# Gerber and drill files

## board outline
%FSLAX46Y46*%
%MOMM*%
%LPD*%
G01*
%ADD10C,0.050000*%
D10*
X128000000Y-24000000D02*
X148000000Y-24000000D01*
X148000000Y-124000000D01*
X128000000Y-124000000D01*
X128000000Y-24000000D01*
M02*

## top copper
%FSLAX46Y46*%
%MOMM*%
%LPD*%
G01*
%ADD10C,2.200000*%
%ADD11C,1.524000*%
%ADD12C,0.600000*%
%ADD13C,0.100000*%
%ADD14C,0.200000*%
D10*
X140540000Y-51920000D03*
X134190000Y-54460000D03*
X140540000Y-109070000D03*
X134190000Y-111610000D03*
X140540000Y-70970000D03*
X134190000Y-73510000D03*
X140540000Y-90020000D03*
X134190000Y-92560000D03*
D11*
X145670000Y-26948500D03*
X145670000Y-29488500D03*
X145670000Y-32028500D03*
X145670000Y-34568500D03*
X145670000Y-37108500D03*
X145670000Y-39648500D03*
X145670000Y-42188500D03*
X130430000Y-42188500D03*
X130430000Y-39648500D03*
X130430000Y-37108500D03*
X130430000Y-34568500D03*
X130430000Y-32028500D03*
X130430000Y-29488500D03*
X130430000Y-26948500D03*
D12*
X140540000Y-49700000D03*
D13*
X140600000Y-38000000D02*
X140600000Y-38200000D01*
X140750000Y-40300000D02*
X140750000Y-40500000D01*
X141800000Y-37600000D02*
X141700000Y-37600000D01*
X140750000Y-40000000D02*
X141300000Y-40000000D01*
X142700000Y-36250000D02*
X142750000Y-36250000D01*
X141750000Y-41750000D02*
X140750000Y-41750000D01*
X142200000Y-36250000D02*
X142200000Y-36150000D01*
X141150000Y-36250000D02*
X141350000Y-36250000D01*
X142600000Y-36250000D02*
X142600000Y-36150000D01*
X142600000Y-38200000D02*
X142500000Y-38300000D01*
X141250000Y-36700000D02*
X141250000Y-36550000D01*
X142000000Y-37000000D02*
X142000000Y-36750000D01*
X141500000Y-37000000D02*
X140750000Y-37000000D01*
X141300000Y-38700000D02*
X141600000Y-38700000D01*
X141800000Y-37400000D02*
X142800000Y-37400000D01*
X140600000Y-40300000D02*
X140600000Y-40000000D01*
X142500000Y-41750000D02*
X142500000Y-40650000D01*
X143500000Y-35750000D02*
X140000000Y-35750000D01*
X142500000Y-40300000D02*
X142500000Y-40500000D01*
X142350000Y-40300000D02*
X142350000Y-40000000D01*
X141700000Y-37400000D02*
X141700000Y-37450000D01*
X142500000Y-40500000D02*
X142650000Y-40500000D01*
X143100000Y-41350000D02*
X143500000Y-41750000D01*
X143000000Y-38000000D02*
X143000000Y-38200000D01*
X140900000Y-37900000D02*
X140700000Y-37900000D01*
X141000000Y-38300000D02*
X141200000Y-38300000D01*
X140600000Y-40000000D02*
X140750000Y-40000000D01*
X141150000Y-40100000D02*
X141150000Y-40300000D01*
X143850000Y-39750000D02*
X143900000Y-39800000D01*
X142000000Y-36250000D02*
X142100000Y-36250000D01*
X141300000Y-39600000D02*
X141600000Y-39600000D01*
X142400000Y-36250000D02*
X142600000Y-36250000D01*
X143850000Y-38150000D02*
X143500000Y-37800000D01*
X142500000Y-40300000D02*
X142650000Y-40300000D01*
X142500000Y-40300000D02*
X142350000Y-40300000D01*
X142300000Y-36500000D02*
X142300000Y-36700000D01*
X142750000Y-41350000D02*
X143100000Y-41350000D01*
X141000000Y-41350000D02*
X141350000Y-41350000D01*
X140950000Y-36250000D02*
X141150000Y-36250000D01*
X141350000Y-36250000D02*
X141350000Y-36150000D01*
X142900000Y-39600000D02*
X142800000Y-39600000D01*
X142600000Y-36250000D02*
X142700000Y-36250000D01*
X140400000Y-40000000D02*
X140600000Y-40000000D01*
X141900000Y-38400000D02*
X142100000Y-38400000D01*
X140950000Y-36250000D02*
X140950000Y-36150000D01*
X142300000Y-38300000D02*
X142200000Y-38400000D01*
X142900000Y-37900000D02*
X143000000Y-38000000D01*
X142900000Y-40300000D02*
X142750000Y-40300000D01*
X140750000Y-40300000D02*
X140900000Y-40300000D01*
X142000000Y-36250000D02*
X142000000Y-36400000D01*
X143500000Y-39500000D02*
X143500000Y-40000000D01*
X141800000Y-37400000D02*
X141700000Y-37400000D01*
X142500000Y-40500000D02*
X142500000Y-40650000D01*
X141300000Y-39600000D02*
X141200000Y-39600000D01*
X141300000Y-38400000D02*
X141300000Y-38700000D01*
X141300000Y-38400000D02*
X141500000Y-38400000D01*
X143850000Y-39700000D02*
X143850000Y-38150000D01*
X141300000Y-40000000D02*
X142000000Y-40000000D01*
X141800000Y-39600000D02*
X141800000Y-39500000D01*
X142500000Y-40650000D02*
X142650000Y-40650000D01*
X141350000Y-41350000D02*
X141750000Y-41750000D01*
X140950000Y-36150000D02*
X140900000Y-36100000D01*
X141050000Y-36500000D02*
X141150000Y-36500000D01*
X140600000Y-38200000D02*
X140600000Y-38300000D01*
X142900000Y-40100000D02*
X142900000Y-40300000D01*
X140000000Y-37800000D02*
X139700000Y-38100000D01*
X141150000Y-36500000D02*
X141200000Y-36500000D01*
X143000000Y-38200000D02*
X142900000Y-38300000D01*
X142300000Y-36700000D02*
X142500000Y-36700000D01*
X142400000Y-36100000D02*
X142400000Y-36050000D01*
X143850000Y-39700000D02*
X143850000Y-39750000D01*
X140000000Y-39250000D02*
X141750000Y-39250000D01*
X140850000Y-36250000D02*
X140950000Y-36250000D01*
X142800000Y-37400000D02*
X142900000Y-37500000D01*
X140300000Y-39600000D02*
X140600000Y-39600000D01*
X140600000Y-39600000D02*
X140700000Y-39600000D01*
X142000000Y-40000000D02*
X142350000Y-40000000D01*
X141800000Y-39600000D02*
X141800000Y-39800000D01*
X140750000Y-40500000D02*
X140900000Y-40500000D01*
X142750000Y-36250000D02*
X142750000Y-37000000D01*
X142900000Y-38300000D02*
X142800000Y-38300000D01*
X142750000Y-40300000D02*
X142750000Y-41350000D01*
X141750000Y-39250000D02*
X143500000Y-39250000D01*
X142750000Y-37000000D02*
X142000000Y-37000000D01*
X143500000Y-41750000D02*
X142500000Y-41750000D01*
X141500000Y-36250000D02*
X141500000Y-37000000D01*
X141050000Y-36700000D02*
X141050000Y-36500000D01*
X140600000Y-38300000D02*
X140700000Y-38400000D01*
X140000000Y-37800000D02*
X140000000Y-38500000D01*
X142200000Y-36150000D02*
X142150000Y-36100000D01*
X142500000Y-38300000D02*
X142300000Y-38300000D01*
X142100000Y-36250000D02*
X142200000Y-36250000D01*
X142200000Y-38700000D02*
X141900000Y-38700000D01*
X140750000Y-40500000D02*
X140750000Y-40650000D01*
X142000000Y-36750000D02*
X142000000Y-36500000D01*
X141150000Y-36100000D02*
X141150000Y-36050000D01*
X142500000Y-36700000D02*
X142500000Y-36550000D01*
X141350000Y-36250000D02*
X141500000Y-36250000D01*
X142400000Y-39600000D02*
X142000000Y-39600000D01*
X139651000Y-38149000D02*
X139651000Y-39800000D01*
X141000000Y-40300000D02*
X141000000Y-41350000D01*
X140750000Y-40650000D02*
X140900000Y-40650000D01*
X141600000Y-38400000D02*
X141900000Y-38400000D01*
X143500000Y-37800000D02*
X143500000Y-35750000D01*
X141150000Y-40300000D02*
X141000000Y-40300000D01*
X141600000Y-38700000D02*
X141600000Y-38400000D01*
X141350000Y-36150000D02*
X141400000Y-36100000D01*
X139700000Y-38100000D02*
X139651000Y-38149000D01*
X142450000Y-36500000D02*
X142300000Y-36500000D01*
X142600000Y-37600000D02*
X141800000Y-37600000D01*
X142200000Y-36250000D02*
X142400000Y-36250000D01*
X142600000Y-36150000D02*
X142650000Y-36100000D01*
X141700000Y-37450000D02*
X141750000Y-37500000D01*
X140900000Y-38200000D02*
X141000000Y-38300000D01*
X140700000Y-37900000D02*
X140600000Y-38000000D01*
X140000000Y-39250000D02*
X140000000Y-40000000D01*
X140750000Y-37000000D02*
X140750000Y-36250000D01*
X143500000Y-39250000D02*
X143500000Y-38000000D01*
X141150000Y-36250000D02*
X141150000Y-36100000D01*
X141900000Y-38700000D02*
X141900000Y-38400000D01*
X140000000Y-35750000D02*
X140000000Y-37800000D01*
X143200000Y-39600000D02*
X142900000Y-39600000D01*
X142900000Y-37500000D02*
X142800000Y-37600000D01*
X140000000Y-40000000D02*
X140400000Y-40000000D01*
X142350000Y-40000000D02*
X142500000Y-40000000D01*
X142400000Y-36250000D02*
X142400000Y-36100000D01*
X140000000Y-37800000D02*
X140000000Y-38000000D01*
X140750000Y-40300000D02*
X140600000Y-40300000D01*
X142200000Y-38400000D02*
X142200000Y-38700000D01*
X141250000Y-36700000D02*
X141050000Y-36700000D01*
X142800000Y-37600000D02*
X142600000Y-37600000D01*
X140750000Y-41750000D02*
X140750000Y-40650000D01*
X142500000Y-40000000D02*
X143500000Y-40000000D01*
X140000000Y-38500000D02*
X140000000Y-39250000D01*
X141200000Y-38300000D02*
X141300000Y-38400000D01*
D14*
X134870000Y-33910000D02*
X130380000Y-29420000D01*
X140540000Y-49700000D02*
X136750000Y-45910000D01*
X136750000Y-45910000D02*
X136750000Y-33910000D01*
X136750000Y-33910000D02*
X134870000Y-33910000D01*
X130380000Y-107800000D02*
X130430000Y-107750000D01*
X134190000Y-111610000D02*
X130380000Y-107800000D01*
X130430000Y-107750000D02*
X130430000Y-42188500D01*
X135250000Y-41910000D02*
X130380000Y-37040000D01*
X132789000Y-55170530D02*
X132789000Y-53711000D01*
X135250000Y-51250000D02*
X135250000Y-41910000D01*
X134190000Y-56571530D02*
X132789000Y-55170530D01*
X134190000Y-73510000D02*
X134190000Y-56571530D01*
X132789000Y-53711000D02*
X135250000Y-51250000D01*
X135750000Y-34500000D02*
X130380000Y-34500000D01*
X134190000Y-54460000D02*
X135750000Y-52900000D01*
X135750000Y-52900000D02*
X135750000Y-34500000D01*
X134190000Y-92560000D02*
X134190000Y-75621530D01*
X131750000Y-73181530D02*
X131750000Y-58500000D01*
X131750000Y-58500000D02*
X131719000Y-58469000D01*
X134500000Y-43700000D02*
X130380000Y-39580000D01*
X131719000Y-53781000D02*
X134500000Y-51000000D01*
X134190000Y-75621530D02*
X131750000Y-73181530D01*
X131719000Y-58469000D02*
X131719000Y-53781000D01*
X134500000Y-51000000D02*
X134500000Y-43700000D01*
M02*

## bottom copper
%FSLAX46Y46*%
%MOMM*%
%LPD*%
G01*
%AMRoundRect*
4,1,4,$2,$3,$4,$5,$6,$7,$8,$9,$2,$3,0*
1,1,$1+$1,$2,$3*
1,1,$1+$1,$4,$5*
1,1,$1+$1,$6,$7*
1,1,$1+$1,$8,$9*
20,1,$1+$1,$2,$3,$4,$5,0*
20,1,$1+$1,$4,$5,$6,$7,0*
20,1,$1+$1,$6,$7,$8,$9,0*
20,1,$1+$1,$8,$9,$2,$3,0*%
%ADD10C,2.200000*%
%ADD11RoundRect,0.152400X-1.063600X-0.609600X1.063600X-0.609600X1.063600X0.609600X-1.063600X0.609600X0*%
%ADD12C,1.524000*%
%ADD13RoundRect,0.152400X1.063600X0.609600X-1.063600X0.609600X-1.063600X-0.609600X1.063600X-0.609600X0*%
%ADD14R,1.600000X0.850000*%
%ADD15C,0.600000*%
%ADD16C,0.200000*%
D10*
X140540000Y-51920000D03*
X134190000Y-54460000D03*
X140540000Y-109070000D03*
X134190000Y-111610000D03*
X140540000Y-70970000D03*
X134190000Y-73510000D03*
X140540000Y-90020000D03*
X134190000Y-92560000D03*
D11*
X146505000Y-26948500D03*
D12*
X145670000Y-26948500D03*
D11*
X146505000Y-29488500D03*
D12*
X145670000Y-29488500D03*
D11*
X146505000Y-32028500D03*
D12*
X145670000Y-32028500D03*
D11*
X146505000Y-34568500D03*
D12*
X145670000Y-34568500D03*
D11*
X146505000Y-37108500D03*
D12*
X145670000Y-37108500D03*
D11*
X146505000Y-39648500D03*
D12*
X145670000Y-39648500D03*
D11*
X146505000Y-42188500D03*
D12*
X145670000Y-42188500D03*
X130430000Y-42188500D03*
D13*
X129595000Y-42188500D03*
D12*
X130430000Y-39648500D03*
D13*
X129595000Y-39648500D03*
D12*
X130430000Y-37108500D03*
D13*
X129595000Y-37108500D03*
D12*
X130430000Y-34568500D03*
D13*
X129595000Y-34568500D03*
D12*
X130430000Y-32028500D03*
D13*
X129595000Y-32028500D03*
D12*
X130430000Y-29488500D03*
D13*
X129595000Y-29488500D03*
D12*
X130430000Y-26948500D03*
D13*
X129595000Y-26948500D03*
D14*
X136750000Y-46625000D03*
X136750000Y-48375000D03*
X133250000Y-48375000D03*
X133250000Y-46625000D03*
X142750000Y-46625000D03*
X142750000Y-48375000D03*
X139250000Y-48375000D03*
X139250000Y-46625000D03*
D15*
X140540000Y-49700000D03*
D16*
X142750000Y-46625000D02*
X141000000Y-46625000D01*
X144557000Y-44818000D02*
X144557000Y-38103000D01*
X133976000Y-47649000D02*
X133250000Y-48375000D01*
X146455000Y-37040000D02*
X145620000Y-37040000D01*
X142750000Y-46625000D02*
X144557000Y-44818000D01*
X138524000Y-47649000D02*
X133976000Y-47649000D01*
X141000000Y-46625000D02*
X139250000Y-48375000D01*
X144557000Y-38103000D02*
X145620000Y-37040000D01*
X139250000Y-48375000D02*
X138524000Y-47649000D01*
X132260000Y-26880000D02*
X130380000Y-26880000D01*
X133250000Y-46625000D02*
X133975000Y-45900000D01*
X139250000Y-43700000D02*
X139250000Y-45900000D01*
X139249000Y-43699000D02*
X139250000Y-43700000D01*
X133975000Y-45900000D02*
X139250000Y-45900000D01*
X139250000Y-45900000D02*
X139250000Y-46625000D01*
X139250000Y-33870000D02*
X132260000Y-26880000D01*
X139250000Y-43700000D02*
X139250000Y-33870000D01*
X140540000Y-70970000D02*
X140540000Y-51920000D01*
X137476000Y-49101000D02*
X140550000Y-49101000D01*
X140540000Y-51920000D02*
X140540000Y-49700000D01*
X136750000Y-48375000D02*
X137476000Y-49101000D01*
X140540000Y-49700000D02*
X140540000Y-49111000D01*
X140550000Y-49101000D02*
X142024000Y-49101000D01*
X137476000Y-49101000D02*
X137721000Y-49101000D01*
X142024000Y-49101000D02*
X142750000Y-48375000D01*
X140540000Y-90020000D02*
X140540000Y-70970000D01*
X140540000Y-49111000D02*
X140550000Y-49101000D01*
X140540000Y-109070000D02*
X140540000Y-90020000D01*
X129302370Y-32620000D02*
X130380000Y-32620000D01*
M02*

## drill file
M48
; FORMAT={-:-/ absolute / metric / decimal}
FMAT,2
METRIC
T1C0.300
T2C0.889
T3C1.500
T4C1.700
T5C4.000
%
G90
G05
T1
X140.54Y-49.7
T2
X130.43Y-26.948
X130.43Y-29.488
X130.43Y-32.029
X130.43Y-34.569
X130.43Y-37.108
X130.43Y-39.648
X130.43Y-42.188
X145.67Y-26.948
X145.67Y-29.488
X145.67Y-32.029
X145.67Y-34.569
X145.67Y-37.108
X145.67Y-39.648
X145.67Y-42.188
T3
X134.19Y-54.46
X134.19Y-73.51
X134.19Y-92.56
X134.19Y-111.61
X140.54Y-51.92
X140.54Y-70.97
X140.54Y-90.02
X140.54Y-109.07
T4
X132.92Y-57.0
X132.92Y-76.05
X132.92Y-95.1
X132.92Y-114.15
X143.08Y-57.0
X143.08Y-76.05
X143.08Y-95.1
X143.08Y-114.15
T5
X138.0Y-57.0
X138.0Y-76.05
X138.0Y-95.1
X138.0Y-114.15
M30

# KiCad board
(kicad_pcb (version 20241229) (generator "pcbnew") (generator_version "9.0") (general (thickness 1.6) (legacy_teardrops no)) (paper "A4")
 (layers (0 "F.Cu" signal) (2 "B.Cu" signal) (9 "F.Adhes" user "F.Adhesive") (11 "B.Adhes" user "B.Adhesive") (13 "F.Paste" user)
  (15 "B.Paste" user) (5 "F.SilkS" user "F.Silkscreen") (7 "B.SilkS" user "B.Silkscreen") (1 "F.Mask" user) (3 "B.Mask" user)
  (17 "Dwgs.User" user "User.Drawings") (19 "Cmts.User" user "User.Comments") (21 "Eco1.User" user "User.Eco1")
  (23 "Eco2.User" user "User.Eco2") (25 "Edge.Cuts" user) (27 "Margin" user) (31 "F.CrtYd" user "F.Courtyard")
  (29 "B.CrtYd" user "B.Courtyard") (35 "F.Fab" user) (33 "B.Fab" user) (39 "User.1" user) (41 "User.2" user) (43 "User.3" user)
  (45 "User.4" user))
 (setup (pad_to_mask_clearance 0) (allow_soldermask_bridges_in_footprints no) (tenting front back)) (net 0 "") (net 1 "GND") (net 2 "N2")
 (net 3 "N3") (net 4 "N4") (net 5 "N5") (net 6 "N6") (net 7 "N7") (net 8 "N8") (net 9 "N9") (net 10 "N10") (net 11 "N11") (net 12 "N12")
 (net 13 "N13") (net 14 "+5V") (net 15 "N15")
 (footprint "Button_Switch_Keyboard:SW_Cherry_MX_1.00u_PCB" (layer "F.Cu") (at 140.54 51.92)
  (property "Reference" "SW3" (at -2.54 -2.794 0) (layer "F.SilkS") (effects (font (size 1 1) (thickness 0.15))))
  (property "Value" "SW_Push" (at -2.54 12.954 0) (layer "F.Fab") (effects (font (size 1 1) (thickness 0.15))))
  (pad "" np_thru_hole circle (at -7.62 5.08) (size 1.7 1.7) (drill 1.7) (layers "*.Cu" "*.Mask"))
  (pad "" np_thru_hole circle (at -2.54 5.08) (size 4 4) (drill 4) (layers "*.Cu" "*.Mask"))
  (pad "" np_thru_hole circle (at 2.54 5.08) (size 1.7 1.7) (drill 1.7) (layers "*.Cu" "*.Mask"))
  (pad "1" thru_hole circle (at 0 0) (size 2.2 2.2) (drill 1.5) (layers "*.Cu" "*.Mask") (remove_unused_layers no) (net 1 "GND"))
  (pad "2" thru_hole circle (at -6.35 2.54) (size 2.2 2.2) (drill 1.5) (layers "*.Cu" "*.Mask") (remove_unused_layers no) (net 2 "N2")))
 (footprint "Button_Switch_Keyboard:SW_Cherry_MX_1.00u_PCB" (layer "F.Cu") (at 140.54 109.07)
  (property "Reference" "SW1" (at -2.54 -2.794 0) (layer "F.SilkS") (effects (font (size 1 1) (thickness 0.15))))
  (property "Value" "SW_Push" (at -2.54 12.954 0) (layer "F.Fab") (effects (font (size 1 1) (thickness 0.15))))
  (pad "" np_thru_hole circle (at -7.62 5.08) (size 1.7 1.7) (drill 1.7) (layers "*.Cu" "*.Mask"))
  (pad "" np_thru_hole circle (at -2.54 5.08) (size 4 4) (drill 4) (layers "*.Cu" "*.Mask"))
  (pad "" np_thru_hole circle (at 2.54 5.08) (size 1.7 1.7) (drill 1.7) (layers "*.Cu" "*.Mask"))
  (pad "1" thru_hole circle (at 0 0) (size 2.2 2.2) (drill 1.5) (layers "*.Cu" "*.Mask") (remove_unused_layers no) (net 1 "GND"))
  (pad "2" thru_hole circle (at -6.35 2.54) (size 2.2 2.2) (drill 1.5) (layers "*.Cu" "*.Mask") (remove_unused_layers no) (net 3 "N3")))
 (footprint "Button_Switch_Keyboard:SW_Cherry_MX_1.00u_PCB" (layer "F.Cu") (at 140.54 70.97)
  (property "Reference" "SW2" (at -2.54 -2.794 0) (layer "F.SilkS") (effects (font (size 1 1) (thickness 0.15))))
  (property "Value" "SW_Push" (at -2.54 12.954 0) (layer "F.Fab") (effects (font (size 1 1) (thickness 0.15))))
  (pad "" np_thru_hole circle (at -7.62 5.08) (size 1.7 1.7) (drill 1.7) (layers "*.Cu" "*.Mask"))
  (pad "" np_thru_hole circle (at -2.54 5.08) (size 4 4) (drill 4) (layers "*.Cu" "*.Mask"))
  (pad "" np_thru_hole circle (at 2.54 5.08) (size 1.7 1.7) (drill 1.7) (layers "*.Cu" "*.Mask"))
  (pad "1" thru_hole circle (at 0 0) (size 2.2 2.2) (drill 1.5) (layers "*.Cu" "*.Mask") (remove_unused_layers no) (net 1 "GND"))
  (pad "2" thru_hole circle (at -6.35 2.54) (size 2.2 2.2) (drill 1.5) (layers "*.Cu" "*.Mask") (remove_unused_layers no) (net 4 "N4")))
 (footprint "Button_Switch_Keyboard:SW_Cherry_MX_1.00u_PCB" (layer "F.Cu") (at 140.54 90.02)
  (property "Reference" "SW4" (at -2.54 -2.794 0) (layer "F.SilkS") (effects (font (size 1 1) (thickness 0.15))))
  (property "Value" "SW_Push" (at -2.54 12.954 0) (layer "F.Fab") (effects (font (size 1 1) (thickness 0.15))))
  (pad "" np_thru_hole circle (at -7.62 5.08) (size 1.7 1.7) (drill 1.7) (layers "*.Cu" "*.Mask"))
  (pad "" np_thru_hole circle (at -2.54 5.08) (size 4 4) (drill 4) (layers "*.Cu" "*.Mask"))
  (pad "" np_thru_hole circle (at 2.54 5.08) (size 1.7 1.7) (drill 1.7) (layers "*.Cu" "*.Mask"))
  (pad "1" thru_hole circle (at 0 0) (size 2.2 2.2) (drill 1.5) (layers "*.Cu" "*.Mask") (remove_unused_layers no) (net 1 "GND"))
  (pad "2" thru_hole circle (at -6.35 2.54) (size 2.2 2.2) (drill 1.5) (layers "*.Cu" "*.Mask") (remove_unused_layers no) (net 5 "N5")))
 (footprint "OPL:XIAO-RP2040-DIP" (layer "B.Cu") (at 138.05 34.5685 180)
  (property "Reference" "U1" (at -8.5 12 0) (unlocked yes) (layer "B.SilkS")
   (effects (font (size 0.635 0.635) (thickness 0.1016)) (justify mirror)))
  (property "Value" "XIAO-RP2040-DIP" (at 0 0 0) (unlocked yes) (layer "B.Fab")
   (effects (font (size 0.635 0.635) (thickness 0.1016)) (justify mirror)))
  (pad "1" smd roundrect (at -8.455 7.62) (size 2.432 1.524) (layers "B.Cu" "B.Mask") (roundrect_rratio 0.1) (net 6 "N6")
   (thermal_bridge_angle 45))
  (pad "1" thru_hole circle (at -7.62 7.62) (size 1.524 1.524) (drill 0.889) (layers "*.Cu" "*.Mask") (remove_unused_layers no) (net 6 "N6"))
  (pad "2" smd roundrect (at -8.455 5.08) (size 2.432 1.524) (layers "B.Cu" "B.Mask") (roundrect_rratio 0.1) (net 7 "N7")
   (thermal_bridge_angle 45))
  (pad "2" thru_hole circle (at -7.62 5.08) (size 1.524 1.524) (drill 0.889) (layers "*.Cu" "*.Mask") (remove_unused_layers no) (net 7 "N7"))
  (pad "3" smd roundrect (at -8.455 2.54) (size 2.432 1.524) (layers "B.Cu" "B.Mask") (roundrect_rratio 0.1) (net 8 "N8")
   (thermal_bridge_angle 45))
  (pad "3" thru_hole circle (at -7.62 2.54) (size 1.524 1.524) (drill 0.889) (layers "*.Cu" "*.Mask") (remove_unused_layers no) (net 8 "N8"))
  (pad "4" smd roundrect (at -8.455 0) (size 2.432 1.524) (layers "B.Cu" "B.Mask") (roundrect_rratio 0.1) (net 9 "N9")
   (thermal_bridge_angle 45))
  (pad "4" thru_hole circle (at -7.62 0) (size 1.524 1.524) (drill 0.889) (layers "*.Cu" "*.Mask") (remove_unused_layers no) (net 9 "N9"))
  (pad "5" smd roundrect (at -8.455 -2.54) (size 2.432 1.524) (layers "B.Cu" "B.Mask") (roundrect_rratio 0.1) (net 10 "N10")
   (thermal_bridge_angle 45))
  (pad "5" thru_hole circle (at -7.62 -2.54) (size 1.524 1.524) (drill 0.889) (layers "*.Cu" "*.Mask") (remove_unused_layers no)
   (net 10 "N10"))
  (pad "6" smd roundrect (at -8.455 -5.08) (size 2.432 1.524) (layers "B.Cu" "B.Mask") (roundrect_rratio 0.1) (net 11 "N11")
   (thermal_bridge_angle 45))
  (pad "6" thru_hole circle (at -7.62 -5.08) (size 1.524 1.524) (drill 0.889) (layers "*.Cu" "*.Mask") (remove_unused_layers no)
   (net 11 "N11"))
  (pad "7" smd roundrect (at -8.455 -7.62) (size 2.432 1.524) (layers "B.Cu" "B.Mask") (roundrect_rratio 0.1) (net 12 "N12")
   (thermal_bridge_angle 45))
  (pad "7" thru_hole circle (at -7.62 -7.62) (size 1.524 1.524) (drill 0.889) (layers "*.Cu" "*.Mask") (remove_unused_layers no)
   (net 12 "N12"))
  (pad "8" thru_hole circle (at 7.62 -7.62 180) (size 1.524 1.524) (drill 0.889) (layers "*.Cu" "*.Mask") (remove_unused_layers no)
   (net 3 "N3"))
  (pad "8" smd roundrect (at 8.455 -7.62 180) (size 2.432 1.524) (layers "B.Cu" "B.Mask") (roundrect_rratio 0.1) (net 3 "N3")
   (thermal_bridge_angle 45))
  (pad "9" thru_hole circle (at 7.62 -5.08 180) (size 1.524 1.524) (drill 0.889) (layers "*.Cu" "*.Mask") (remove_unused_layers no)
   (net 5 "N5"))
  (pad "9" smd roundrect (at 8.455 -5.08 180) (size 2.432 1.524) (layers "B.Cu" "B.Mask") (roundrect_rratio 0.1) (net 5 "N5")
   (thermal_bridge_angle 45))
  (pad "10" thru_hole circle (at 7.62 -2.54 180) (size 1.524 1.524) (drill 0.889) (layers "*.Cu" "*.Mask") (remove_unused_layers no)
   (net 4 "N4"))
  (pad "10" smd roundrect (at 8.455 -2.54 180) (size 2.432 1.524) (layers "B.Cu" "B.Mask") (roundrect_rratio 0.1) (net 4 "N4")
   (thermal_bridge_angle 45))
  (pad "11" thru_hole circle (at 7.62 0 180) (size 1.524 1.524) (drill 0.889) (layers "*.Cu" "*.Mask") (remove_unused_layers no)
   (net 2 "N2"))
  (pad "11" smd roundrect (at 8.455 0 180) (size 2.432 1.524) (layers "B.Cu" "B.Mask") (roundrect_rratio 0.1) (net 2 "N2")
   (thermal_bridge_angle 45))
  (pad "12" thru_hole circle (at 7.62 2.54 180) (size 1.524 1.524) (drill 0.889) (layers "*.Cu" "*.Mask") (remove_unused_layers no)
   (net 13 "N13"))
  (pad "12" smd roundrect (at 8.455 2.54 180) (size 2.432 1.524) (layers "B.Cu" "B.Mask") (roundrect_rratio 0.1) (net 13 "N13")
   (thermal_bridge_angle 45))
  (pad "13" thru_hole circle (at 7.62 5.08 180) (size 1.524 1.524) (drill 0.889) (layers "*.Cu" "*.Mask") (remove_unused_layers no)
   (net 1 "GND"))
  (pad "13" smd roundrect (at 8.455 5.08 180) (size 2.432 1.524) (layers "B.Cu" "B.Mask") (roundrect_rratio 0.1) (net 1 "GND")
   (thermal_bridge_angle 45))
  (pad "14" thru_hole circle (at 7.62 7.62 180) (size 1.524 1.524) (drill 0.889) (layers "*.Cu" "*.Mask") (remove_unused_layers no)
   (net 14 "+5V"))
  (pad "14" smd roundrect (at 8.455 7.62 180) (size 2.432 1.524) (layers "B.Cu" "B.Mask") (roundrect_rratio 0.1) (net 14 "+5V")
   (thermal_bridge_angle 45)))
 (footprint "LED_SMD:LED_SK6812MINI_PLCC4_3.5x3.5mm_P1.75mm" (layer "B.Cu") (at 135 47.5 180)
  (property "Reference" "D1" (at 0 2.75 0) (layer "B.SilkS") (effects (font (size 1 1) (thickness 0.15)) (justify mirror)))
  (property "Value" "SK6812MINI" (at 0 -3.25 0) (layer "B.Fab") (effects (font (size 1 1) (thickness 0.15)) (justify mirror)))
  (pad "1" smd rect (at -1.75 0.875 180) (size 1.6 0.85) (layers "B.Cu" "B.Mask" "B.Paste") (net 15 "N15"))
  (pad "2" smd rect (at -1.75 -0.875 180) (size 1.6 0.85) (layers "B.Cu" "B.Mask" "B.Paste") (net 1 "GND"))
  (pad "3" smd rect (at 1.75 -0.875 180) (size 1.6 0.85) (layers "B.Cu" "B.Mask" "B.Paste") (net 10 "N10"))
  (pad "4" smd rect (at 1.75 0.875 180) (size 1.6 0.85) (layers "B.Cu" "B.Mask" "B.Paste") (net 14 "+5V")))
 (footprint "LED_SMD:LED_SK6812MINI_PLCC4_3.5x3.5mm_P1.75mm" (layer "B.Cu") (at 141 47.5 180)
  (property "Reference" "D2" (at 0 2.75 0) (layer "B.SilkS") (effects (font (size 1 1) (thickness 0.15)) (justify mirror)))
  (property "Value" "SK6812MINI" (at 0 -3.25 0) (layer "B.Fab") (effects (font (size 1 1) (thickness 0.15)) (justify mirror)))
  (pad "1" smd rect (at -1.75 0.875 180) (size 1.6 0.85) (layers "B.Cu" "B.Mask" "B.Paste") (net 10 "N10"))
  (pad "2" smd rect (at -1.75 -0.875 180) (size 1.6 0.85) (layers "B.Cu" "B.Mask" "B.Paste") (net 1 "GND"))
  (pad "3" smd rect (at 1.75 -0.875 180) (size 1.6 0.85) (layers "B.Cu" "B.Mask" "B.Paste") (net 10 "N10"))
  (pad "4" smd rect (at 1.75 0.875 180) (size 1.6 0.85) (layers "B.Cu" "B.Mask" "B.Paste") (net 14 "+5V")))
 (gr_rect (start 128 24) (end 148 124) (stroke (width 0.05) (type default)) (fill no) (layer "Edge.Cuts"))
 (segment (start 140.6 38) (end 140.6 38.2) (width 0.1) (layer "F.Cu") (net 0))
 (segment (start 140.75 40.3) (end 140.75 40.5) (width 0.1) (layer "F.Cu") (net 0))
 (segment (start 141.8 37.6) (end 141.7 37.6) (width 0.1) (layer "F.Cu") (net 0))
 (segment (start 140.75 40) (end 141.3 40) (width 0.1) (layer "F.Cu") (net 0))
 (segment (start 142.7 36.25) (end 142.75 36.25) (width 0.1) (layer "F.Cu") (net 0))
 (segment (start 141.75 41.75) (end 140.75 41.75) (width 0.1) (layer "F.Cu") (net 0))
 (segment (start 142.2 36.25) (end 142.2 36.15) (width 0.1) (layer "F.Cu") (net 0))
 (segment (start 141.15 36.25) (end 141.35 36.25) (width 0.1) (layer "F.Cu") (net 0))
 (segment (start 142.6 36.25) (end 142.6 36.15) (width 0.1) (layer "F.Cu") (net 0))
 (segment (start 142.6 38.2) (end 142.5 38.3) (width 0.1) (layer "F.Cu") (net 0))
 (segment (start 141.25 36.7) (end 141.25 36.55) (width 0.1) (layer "F.Cu") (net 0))
 (segment (start 142 37) (end 142 36.75) (width 0.1) (layer "F.Cu") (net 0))
 (segment (start 141.5 37) (end 140.75 37) (width 0.1) (layer "F.Cu") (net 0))
 (segment (start 141.3 38.7) (end 141.6 38.7) (width 0.1) (layer "F.Cu") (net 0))
 (segment (start 141.8 37.4) (end 142.8 37.4) (width 0.1) (layer "F.Cu") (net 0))
 (segment (start 140.6 40.3) (end 140.6 40) (width 0.1) (layer "F.Cu") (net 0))
 (segment (start 142.5 41.75) (end 142.5 40.65) (width 0.1) (layer "F.Cu") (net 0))
 (segment (start 143.5 35.75) (end 140 35.75) (width 0.1) (layer "F.Cu") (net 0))
 (segment (start 142.5 40.3) (end 142.5 40.5) (width 0.1) (layer "F.Cu") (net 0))
 (segment (start 142.35 40.3) (end 142.35 40) (width 0.1) (layer "F.Cu") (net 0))
 (segment (start 141.7 37.4) (end 141.7 37.45) (width 0.1) (layer "F.Cu") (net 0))
 (segment (start 142.5 40.5) (end 142.65 40.5) (width 0.1) (layer "F.Cu") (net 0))
 (segment (start 143.1 41.35) (end 143.5 41.75) (width 0.1) (layer "F.Cu") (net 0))
 (segment (start 143 38) (end 143 38.2) (width 0.1) (layer "F.Cu") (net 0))
 (segment (start 140.9 37.9) (end 140.7 37.9) (width 0.1) (layer "F.Cu") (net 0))
 (segment (start 141 38.3) (end 141.2 38.3) (width 0.1) (layer "F.Cu") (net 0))
 (segment (start 140.6 40) (end 140.75 40) (width 0.1) (layer "F.Cu") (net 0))
 (segment (start 141.15 40.1) (end 141.15 40.3) (width 0.1) (layer "F.Cu") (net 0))
 (segment (start 143.85 39.75) (end 143.9 39.8) (width 0.1) (layer "F.Cu") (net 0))
 (segment (start 142 36.25) (end 142.1 36.25) (width 0.1) (layer "F.Cu") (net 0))
 (segment (start 141.3 39.6) (end 141.6 39.6) (width 0.1) (layer "F.Cu") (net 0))
 (segment (start 142.4 36.25) (end 142.6 36.25) (width 0.1) (layer "F.Cu") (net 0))
 (segment (start 143.85 38.15) (end 143.5 37.8) (width 0.1) (layer "F.Cu") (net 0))
 (segment (start 142.5 40.3) (end 142.65 40.3) (width 0.1) (layer "F.Cu") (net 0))
 (segment (start 142.5 40.3) (end 142.35 40.3) (width 0.1) (layer "F.Cu") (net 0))
 (segment (start 142.3 36.5) (end 142.3 36.7) (width 0.1) (layer "F.Cu") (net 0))
 (segment (start 142.75 41.35) (end 143.1 41.35) (width 0.1) (layer "F.Cu") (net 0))
 (segment (start 141 41.35) (end 141.35 41.35) (width 0.1) (layer "F.Cu") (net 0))
 (segment (start 140.95 36.25) (end 141.15 36.25) (width 0.1) (layer "F.Cu") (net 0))
 (segment (start 141.35 36.25) (end 141.35 36.15) (width 0.1) (layer "F.Cu") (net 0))
 (segment (start 142.9 39.6) (end 142.8 39.6) (width 0.1) (layer "F.Cu") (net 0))
 (segment (start 142.6 36.25) (end 142.7 36.25) (width 0.1) (layer "F.Cu") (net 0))
 (segment (start 140.4 40) (end 140.6 40) (width 0.1) (layer "F.Cu") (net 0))
 (segment (start 141.9 38.4) (end 142.1 38.4) (width 0.1) (layer "F.Cu") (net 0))
 (segment (start 140.95 36.25) (end 140.95 36.15) (width 0.1) (layer "F.Cu") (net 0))
 (segment (start 142.3 38.3) (end 142.2 38.4) (width 0.1) (layer "F.Cu") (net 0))
 (segment (start 142.9 37.9) (end 143 38) (width 0.1) (layer "F.Cu") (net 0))
 (segment (start 142.9 40.3) (end 142.75 40.3) (width 0.1) (layer "F.Cu") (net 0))
 (segment (start 140.75 40.3) (end 140.9 40.3) (width 0.1) (layer "F.Cu") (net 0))
 (segment (start 142 36.25) (end 142 36.4) (width 0.1) (layer "F.Cu") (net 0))
 (segment (start 143.5 39.5) (end 143.5 40) (width 0.1) (layer "F.Cu") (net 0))
 (segment (start 141.8 37.4) (end 141.7 37.4) (width 0.1) (layer "F.Cu") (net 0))
 (segment (start 142.5 40.5) (end 142.5 40.65) (width 0.1) (layer "F.Cu") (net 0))
 (segment (start 141.3 39.6) (end 141.2 39.6) (width 0.1) (layer "F.Cu") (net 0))
 (segment (start 141.3 38.4) (end 141.3 38.7) (width 0.1) (layer "F.Cu") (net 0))
 (segment (start 141.3 38.4) (end 141.5 38.4) (width 0.1) (layer "F.Cu") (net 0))
 (segment (start 143.85 39.7) (end 143.85 38.15) (width 0.1) (layer "F.Cu") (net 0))
 (segment (start 141.3 40) (end 142 40) (width 0.1) (layer "F.Cu") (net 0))
 (segment (start 141.8 39.6) (end 141.8 39.5) (width 0.1) (layer "F.Cu") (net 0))
 (segment (start 142.5 40.65) (end 142.65 40.65) (width 0.1) (layer "F.Cu") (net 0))
 (segment (start 141.35 41.35) (end 141.75 41.75) (width 0.1) (layer "F.Cu") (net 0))
 (segment (start 140.95 36.15) (end 140.9 36.1) (width 0.1) (layer "F.Cu") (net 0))
 (segment (start 141.05 36.5) (end 141.15 36.5) (width 0.1) (layer "F.Cu") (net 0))
 (segment (start 140.6 38.2) (end 140.6 38.3) (width 0.1) (layer "F.Cu") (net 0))
 (segment (start 142.9 40.1) (end 142.9 40.3) (width 0.1) (layer "F.Cu") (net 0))
 (segment (start 140 37.8) (end 139.7 38.1) (width 0.1) (layer "F.Cu") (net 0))
 (segment (start 141.15 36.5) (end 141.2 36.5) (width 0.1) (layer "F.Cu") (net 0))
 (segment (start 143 38.2) (end 142.9 38.3) (width 0.1) (layer "F.Cu") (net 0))
 (segment (start 142.3 36.7) (end 142.5 36.7) (width 0.1) (layer "F.Cu") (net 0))
 (segment (start 142.4 36.1) (end 142.4 36.05) (width 0.1) (layer "F.Cu") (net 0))
 (segment (start 143.85 39.7) (end 143.85 39.75) (width 0.1) (layer "F.Cu") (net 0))
 (segment (start 140 39.25) (end 141.75 39.25) (width 0.1) (layer "F.Cu") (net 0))
 (segment (start 140.85 36.25) (end 140.95 36.25) (width 0.1) (layer "F.Cu") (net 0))
 (segment (start 142.8 37.4) (end 142.9 37.5) (width 0.1) (layer "F.Cu") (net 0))
 (segment (start 140.3 39.6) (end 140.6 39.6) (width 0.1) (layer "F.Cu") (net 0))
 (segment (start 140.6 39.6) (end 140.7 39.6) (width 0.1) (layer "F.Cu") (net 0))
 (segment (start 142 40) (end 142.35 40) (width 0.1) (layer "F.Cu") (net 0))
 (segment (start 141.8 39.6) (end 141.8 39.8) (width 0.1) (layer "F.Cu") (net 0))
 (segment (start 140.75 40.5) (end 140.9 40.5) (width 0.1) (layer "F.Cu") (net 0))
 (segment (start 142.75 36.25) (end 142.75 37) (width 0.1) (layer "F.Cu") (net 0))
 (segment (start 142.9 38.3) (end 142.8 38.3) (width 0.1) (layer "F.Cu") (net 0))
 (segment (start 142.75 40.3) (end 142.75 41.35) (width 0.1) (layer "F.Cu") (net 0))
 (segment (start 141.75 39.25) (end 143.5 39.25) (width 0.1) (layer "F.Cu") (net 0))
 (segment (start 142.75 37) (end 142 37) (width 0.1) (layer "F.Cu") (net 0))
 (segment (start 143.5 41.75) (end 142.5 41.75) (width 0.1) (layer "F.Cu") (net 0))
 (segment (start 141.5 36.25) (end 141.5 37) (width 0.1) (layer "F.Cu") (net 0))
 (segment (start 141.05 36.7) (end 141.05 36.5) (width 0.1) (layer "F.Cu") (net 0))
 (segment (start 140.6 38.3) (end 140.7 38.4) (width 0.1) (layer "F.Cu") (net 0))
 (segment (start 140 37.8) (end 140 38.5) (width 0.1) (layer "F.Cu") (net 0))
 (segment (start 142.2 36.15) (end 142.15 36.1) (width 0.1) (layer "F.Cu") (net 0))
 (segment (start 142.5 38.3) (end 142.3 38.3) (width 0.1) (layer "F.Cu") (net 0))
 (segment (start 142.1 36.25) (end 142.2 36.25) (width 0.1) (layer "F.Cu") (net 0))
 (segment (start 142.2 38.7) (end 141.9 38.7) (width 0.1) (layer "F.Cu") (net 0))
 (segment (start 140.75 40.5) (end 140.75 40.65) (width 0.1) (layer "F.Cu") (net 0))
 (segment (start 142 36.75) (end 142 36.5) (width 0.1) (layer "F.Cu") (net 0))
 (segment (start 141.15 36.1) (end 141.15 36.05) (width 0.1) (layer "F.Cu") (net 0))
 (segment (start 142.5 36.7) (end 142.5 36.55) (width 0.1) (layer "F.Cu") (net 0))
 (segment (start 141.35 36.25) (end 141.5 36.25) (width 0.1) (layer "F.Cu") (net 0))
 (segment (start 142.4 39.6) (end 142 39.6) (width 0.1) (layer "F.Cu") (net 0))
 (segment (start 139.651 38.149) (end 139.651 39.8) (width 0.1) (layer "F.Cu") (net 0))
 (segment (start 141 40.3) (end 141 41.35) (width 0.1) (layer "F.Cu") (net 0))
 (segment (start 140.75 40.65) (end 140.9 40.65) (width 0.1) (layer "F.Cu") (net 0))
 (segment (start 141.6 38.4) (end 141.9 38.4) (width 0.1) (layer "F.Cu") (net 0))
 (segment (start 143.5 37.8) (end 143.5 35.75) (width 0.1) (layer "F.Cu") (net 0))
 (segment (start 141.15 40.3) (end 141 40.3) (width 0.1) (layer "F.Cu") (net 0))
 (segment (start 141.6 38.7) (end 141.6 38.4) (width 0.1) (layer "F.Cu") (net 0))
 (segment (start 141.35 36.15) (end 141.4 36.1) (width 0.1) (layer "F.Cu") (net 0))
 (segment (start 139.7 38.1) (end 139.651 38.149) (width 0.1) (layer "F.Cu") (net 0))
 (segment (start 142.45 36.5) (end 142.3 36.5) (width 0.1) (layer "F.Cu") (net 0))
 (segment (start 142.6 37.6) (end 141.8 37.6) (width 0.1) (layer "F.Cu") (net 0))
 (segment (start 142.2 36.25) (end 142.4 36.25) (width 0.1) (layer "F.Cu") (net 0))
 (segment (start 142.6 36.15) (end 142.65 36.1) (width 0.1) (layer "F.Cu") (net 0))
 (segment (start 141.7 37.45) (end 141.75 37.5) (width 0.1) (layer "F.Cu") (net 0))
 (segment (start 140.9 38.2) (end 141 38.3) (width 0.1) (layer "F.Cu") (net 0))
 (segment (start 140.7 37.9) (end 140.6 38) (width 0.1) (layer "F.Cu") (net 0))
 (segment (start 140 39.25) (end 140 40) (width 0.1) (layer "F.Cu") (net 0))
 (segment (start 140.75 37) (end 140.75 36.25) (width 0.1) (layer "F.Cu") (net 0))
 (segment (start 143.5 39.25) (end 143.5 38) (width 0.1) (layer "F.Cu") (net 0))
 (segment (start 141.15 36.25) (end 141.15 36.1) (width 0.1) (layer "F.Cu") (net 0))
 (segment (start 141.9 38.7) (end 141.9 38.4) (width 0.1) (layer "F.Cu") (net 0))
 (segment (start 140 35.75) (end 140 37.8) (width 0.1) (layer "F.Cu") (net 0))
 (segment (start 143.2 39.6) (end 142.9 39.6) (width 0.1) (layer "F.Cu") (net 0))
 (segment (start 142.9 37.5) (end 142.8 37.6) (width 0.1) (layer "F.Cu") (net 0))
 (segment (start 140 40) (end 140.4 40) (width 0.1) (layer "F.Cu") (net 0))
 (segment (start 142.35 40) (end 142.5 40) (width 0.1) (layer "F.Cu") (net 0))
 (segment (start 142.4 36.25) (end 142.4 36.1) (width 0.1) (layer "F.Cu") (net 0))
 (segment (start 140 37.8) (end 140 38) (width 0.1) (layer "F.Cu") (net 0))
 (segment (start 140.75 40.3) (end 140.6 40.3) (width 0.1) (layer "F.Cu") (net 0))
 (segment (start 142.2 38.4) (end 142.2 38.7) (width 0.1) (layer "F.Cu") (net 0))
 (segment (start 141.25 36.7) (end 141.05 36.7) (width 0.1) (layer "F.Cu") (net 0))
 (segment (start 142.8 37.6) (end 142.6 37.6) (width 0.1) (layer "F.Cu") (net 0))
 (segment (start 140.75 41.75) (end 140.75 40.65) (width 0.1) (layer "F.Cu") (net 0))
 (segment (start 142.5 40) (end 143.5 40) (width 0.1) (layer "F.Cu") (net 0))
 (segment (start 140 38.5) (end 140 39.25) (width 0.1) (layer "F.Cu") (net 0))
 (segment (start 141.2 38.3) (end 141.3 38.4) (width 0.1) (layer "F.Cu") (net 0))
 (segment (start 142.75 46.625) (end 141 46.625) (width 0.2) (layer "B.Cu") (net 10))
 (segment (start 144.557 44.818) (end 144.557 38.103) (width 0.2) (layer "B.Cu") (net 10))
 (segment (start 133.976 47.649) (end 133.25 48.375) (width 0.2) (layer "B.Cu") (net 10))
 (segment (start 146.455 37.04) (end 145.62 37.04) (width 0.2) (layer "B.Cu") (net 10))
 (segment (start 142.75 46.625) (end 144.557 44.818) (width 0.2) (layer "B.Cu") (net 10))
 (segment (start 138.524 47.649) (end 133.976 47.649) (width 0.2) (layer "B.Cu") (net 10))
 (segment (start 141 46.625) (end 139.25 48.375) (width 0.2) (layer "B.Cu") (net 10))
 (segment (start 144.557 38.103) (end 145.62 37.04) (width 0.2) (layer "B.Cu") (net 10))
 (segment (start 139.25 48.375) (end 138.524 47.649) (width 0.2) (layer "B.Cu") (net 10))
 (segment (start 132.26 26.88) (end 130.38 26.88) (width 0.2) (layer "B.Cu") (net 14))
 (segment (start 133.25 46.625) (end 133.975 45.9) (width 0.2) (layer "B.Cu") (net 14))
 (segment (start 139.25 43.7) (end 139.25 45.9) (width 0.2) (layer "B.Cu") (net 14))
 (segment (start 139.249 43.699) (end 139.25 43.7) (width 0.2) (layer "B.Cu") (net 14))
 (segment (start 133.975 45.9) (end 139.25 45.9) (width 0.2) (layer "B.Cu") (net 14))
 (segment (start 139.25 45.9) (end 139.25 46.625) (width 0.2) (layer "B.Cu") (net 14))
 (segment (start 139.25 33.87) (end 132.26 26.88) (width 0.2) (layer "B.Cu") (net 14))
 (segment (start 139.25 43.7) (end 139.25 33.87) (width 0.2) (layer "B.Cu") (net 14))
 (segment (start 134.87 33.91) (end 130.38 29.42) (width 0.2) (layer "F.Cu") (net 1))
 (segment (start 140.54 49.7) (end 136.75 45.91) (width 0.2) (layer "F.Cu") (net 1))
 (segment (start 136.75 45.91) (end 136.75 33.91) (width 0.2) (layer "F.Cu") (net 1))
 (segment (start 136.75 33.91) (end 134.87 33.91) (width 0.2) (layer "F.Cu") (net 1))
 (via (at 140.54 49.7) (size 0.6) (drill 0.3) (layers "F.Cu" "B.Cu") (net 1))
 (segment (start 140.54 70.97) (end 140.54 51.92) (width 0.2) (layer "B.Cu") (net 1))
 (segment (start 137.476 49.101) (end 140.55 49.101) (width 0.2) (layer "B.Cu") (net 1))
 (segment (start 140.54 51.92) (end 140.54 49.7) (width 0.2) (layer "B.Cu") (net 1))
 (segment (start 136.75 48.375) (end 137.476 49.101) (width 0.2) (layer "B.Cu") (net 1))
 (segment (start 140.54 49.7) (end 140.54 49.111) (width 0.2) (layer "B.Cu") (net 1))
 (segment (start 140.55 49.101) (end 142.024 49.101) (width 0.2) (layer "B.Cu") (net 1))
 (segment (start 137.476 49.101) (end 137.721 49.101) (width 0.2) (layer "B.Cu") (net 1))
 (segment (start 142.024 49.101) (end 142.75 48.375) (width 0.2) (layer "B.Cu") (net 1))
 (segment (start 140.54 90.02) (end 140.54 70.97) (width 0.2) (layer "B.Cu") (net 1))
 (segment (start 140.54 49.111) (end 140.55 49.101) (width 0.2) (layer "B.Cu") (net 1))
 (segment (start 140.54 109.07) (end 140.54 90.02) (width 0.2) (layer "B.Cu") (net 1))
 (segment (start 130.38 107.8) (end 130.43 107.75) (width 0.2) (layer "F.Cu") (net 3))
 (segment (start 134.19 111.61) (end 130.38 107.8) (width 0.2) (layer "F.Cu") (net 3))
 (segment (start 130.43 107.75) (end 130.43 42.1885) (width 0.2) (layer "F.Cu") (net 3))
 (segment (start 135.25 41.91) (end 130.38 37.04) (width 0.2) (layer "F.Cu") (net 4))
 (segment (start 132.789 55.17053) (end 132.789 53.711) (width 0.2) (layer "F.Cu") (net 4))
 (segment (start 135.25 51.25) (end 135.25 41.91) (width 0.2) (layer "F.Cu") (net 4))
 (segment (start 134.19 56.57153) (end 132.789 55.17053) (width 0.2) (layer "F.Cu") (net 4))
 (segment (start 134.19 73.51) (end 134.19 56.57153) (width 0.2) (layer "F.Cu") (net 4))
 (segment (start 132.789 53.711) (end 135.25 51.25) (width 0.2) (layer "F.Cu") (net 4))
 (segment (start 135.75 34.5) (end 130.38 34.5) (width 0.2) (layer "F.Cu") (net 2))
 (segment (start 134.19 54.46) (end 135.75 52.9) (width 0.2) (layer "F.Cu") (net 2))
 (segment (start 135.75 52.9) (end 135.75 34.5) (width 0.2) (layer "F.Cu") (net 2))
 (segment (start 134.19 92.56) (end 134.19 75.62153) (width 0.2) (layer "F.Cu") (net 5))
 (segment (start 131.75 73.18153) (end 131.75 58.5) (width 0.2) (layer "F.Cu") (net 5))
 (segment (start 131.75 58.5) (end 131.719 58.469) (width 0.2) (layer "F.Cu") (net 5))
 (segment (start 134.5 43.7) (end 130.38 39.58) (width 0.2) (layer "F.Cu") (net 5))
 (segment (start 131.719 53.781) (end 134.5 51) (width 0.2) (layer "F.Cu") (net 5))
 (segment (start 134.19 75.62153) (end 131.75 73.18153) (width 0.2) (layer "F.Cu") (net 5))
 (segment (start 131.719 58.469) (end 131.719 53.781) (width 0.2) (layer "F.Cu") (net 5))
 (segment (start 134.5 51) (end 134.5 43.7) (width 0.2) (layer "F.Cu") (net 5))
 (segment (start 129.30237 32.62) (end 130.38 32.62) (width 0.2) (layer "B.Cu") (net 13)))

